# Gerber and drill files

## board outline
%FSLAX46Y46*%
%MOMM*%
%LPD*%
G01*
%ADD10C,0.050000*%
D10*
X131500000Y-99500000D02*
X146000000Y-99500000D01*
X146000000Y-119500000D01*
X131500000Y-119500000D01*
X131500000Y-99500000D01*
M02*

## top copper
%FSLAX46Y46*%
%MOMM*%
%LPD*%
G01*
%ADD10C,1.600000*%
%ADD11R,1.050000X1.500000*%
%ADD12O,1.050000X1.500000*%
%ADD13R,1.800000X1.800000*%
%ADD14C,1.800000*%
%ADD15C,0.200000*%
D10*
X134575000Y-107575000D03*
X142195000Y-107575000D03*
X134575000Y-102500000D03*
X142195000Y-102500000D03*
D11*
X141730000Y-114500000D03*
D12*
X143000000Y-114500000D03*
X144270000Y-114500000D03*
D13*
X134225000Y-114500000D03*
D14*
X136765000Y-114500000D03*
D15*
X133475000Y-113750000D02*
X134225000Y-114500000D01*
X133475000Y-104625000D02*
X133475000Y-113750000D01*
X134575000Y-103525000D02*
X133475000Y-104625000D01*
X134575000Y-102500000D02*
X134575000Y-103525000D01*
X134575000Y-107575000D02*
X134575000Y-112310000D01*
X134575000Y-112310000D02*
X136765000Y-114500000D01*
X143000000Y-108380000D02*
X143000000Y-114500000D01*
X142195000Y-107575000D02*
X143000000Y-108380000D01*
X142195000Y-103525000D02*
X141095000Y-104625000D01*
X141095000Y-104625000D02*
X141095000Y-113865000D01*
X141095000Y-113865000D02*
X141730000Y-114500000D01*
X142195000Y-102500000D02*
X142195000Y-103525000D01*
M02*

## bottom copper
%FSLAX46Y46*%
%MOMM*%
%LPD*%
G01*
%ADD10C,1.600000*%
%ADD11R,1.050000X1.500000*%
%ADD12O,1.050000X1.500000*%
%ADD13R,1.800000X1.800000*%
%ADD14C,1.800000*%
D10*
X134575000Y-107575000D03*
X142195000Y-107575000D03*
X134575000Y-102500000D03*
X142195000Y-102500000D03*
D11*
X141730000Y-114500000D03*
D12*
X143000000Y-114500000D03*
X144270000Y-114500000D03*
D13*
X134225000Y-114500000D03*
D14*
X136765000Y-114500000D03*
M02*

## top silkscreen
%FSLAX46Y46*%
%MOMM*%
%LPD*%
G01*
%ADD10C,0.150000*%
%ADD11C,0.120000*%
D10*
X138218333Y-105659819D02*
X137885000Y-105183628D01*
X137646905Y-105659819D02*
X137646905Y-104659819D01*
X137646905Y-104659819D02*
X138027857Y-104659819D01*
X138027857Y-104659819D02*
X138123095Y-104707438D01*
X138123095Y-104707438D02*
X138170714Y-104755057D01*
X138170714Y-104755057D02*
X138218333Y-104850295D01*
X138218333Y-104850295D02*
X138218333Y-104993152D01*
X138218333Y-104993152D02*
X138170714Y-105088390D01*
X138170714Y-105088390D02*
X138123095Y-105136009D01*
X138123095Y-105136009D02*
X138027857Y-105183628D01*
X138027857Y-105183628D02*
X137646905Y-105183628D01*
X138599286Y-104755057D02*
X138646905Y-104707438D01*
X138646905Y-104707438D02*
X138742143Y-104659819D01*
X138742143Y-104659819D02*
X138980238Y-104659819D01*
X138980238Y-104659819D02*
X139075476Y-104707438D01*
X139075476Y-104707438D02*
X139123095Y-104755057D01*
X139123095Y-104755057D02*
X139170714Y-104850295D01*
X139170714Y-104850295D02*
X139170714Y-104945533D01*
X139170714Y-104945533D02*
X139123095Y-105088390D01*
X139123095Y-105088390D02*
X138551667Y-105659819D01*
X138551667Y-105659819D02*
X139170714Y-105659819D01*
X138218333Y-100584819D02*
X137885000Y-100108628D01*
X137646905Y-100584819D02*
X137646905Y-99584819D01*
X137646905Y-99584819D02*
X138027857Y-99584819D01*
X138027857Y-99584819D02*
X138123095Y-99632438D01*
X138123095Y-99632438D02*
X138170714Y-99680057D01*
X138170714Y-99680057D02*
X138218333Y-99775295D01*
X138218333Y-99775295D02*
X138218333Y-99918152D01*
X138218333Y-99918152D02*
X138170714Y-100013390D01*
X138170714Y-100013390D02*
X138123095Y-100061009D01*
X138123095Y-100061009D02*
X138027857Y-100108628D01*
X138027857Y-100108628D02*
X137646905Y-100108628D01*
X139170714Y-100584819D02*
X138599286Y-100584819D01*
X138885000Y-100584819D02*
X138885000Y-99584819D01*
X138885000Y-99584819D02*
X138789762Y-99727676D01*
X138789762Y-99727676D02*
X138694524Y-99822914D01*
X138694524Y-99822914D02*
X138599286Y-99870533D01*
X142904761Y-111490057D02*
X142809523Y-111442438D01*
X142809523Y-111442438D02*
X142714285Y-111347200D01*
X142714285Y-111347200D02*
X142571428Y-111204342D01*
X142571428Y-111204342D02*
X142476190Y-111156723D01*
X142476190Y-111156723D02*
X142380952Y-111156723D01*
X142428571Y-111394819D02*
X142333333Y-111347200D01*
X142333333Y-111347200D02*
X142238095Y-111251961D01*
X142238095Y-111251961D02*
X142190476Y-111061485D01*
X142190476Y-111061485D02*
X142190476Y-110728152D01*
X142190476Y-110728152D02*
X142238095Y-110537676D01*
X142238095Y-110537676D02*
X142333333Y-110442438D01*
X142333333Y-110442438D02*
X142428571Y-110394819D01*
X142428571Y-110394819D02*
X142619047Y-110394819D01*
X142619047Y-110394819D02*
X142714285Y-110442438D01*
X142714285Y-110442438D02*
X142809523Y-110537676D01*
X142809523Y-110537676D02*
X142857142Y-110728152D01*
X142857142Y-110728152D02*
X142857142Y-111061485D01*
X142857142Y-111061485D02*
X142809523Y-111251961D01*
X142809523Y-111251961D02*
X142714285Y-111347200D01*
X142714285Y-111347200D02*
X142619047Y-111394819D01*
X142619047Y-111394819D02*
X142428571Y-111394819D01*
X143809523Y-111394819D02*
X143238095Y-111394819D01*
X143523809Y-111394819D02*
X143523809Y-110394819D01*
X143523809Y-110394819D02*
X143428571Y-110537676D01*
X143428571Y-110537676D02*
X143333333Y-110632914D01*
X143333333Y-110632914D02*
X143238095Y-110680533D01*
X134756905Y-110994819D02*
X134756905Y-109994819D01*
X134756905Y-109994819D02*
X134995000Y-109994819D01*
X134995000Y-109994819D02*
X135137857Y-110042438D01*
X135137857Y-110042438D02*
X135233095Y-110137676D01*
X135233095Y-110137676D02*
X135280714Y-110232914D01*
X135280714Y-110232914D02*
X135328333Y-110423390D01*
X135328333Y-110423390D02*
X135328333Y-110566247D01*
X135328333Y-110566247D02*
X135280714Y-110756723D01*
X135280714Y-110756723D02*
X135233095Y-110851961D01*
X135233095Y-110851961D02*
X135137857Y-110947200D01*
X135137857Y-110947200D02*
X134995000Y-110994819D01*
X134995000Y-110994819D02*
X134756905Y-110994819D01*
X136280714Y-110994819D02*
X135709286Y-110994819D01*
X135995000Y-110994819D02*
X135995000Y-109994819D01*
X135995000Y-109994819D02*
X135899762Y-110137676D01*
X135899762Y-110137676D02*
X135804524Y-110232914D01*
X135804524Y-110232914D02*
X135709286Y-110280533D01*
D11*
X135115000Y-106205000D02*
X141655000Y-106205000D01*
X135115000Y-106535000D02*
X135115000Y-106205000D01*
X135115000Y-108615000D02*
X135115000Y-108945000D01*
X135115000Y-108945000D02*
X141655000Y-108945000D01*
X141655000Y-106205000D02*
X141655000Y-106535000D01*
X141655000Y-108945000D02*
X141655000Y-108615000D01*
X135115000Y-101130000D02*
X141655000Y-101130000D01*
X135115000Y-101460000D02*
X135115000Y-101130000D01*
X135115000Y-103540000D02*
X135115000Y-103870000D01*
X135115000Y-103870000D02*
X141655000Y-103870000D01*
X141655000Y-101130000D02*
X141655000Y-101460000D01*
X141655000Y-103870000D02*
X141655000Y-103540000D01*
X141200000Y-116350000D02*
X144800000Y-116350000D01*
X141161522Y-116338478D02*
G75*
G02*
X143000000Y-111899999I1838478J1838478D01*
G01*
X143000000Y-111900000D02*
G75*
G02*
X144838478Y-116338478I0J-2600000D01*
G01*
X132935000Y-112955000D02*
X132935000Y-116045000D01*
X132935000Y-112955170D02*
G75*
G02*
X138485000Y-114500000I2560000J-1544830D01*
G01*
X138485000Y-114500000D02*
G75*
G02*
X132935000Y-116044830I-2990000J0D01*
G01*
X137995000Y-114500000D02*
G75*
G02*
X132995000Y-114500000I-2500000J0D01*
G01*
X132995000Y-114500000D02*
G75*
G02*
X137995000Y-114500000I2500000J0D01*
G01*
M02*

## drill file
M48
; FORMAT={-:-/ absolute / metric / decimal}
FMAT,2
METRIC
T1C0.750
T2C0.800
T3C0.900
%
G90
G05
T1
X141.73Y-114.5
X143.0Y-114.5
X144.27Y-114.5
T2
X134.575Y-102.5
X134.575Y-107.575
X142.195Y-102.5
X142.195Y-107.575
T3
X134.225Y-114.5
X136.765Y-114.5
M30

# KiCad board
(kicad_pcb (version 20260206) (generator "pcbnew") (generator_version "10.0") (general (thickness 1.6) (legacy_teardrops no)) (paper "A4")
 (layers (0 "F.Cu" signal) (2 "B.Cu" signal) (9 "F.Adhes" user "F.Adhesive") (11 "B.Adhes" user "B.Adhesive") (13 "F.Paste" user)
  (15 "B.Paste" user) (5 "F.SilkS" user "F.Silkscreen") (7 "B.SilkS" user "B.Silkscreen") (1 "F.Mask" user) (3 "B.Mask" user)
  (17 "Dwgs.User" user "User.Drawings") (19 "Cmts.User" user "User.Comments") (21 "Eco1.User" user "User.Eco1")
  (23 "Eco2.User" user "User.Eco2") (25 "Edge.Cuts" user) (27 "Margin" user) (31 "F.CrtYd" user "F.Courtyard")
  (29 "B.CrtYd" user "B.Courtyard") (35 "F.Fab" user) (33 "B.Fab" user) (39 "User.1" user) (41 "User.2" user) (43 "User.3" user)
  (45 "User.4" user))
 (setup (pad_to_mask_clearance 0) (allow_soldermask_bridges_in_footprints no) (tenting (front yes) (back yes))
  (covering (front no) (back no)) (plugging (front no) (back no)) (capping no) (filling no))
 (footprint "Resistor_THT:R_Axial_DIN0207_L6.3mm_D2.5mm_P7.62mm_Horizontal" (layer "F.Cu") (at 134.575 107.575)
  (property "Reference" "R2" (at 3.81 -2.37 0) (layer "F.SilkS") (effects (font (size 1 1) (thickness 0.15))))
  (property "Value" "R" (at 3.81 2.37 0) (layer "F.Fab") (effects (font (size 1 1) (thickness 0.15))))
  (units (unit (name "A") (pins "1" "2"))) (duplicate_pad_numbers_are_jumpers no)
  (fp_line (start 0.54 -1.37) (end 7.08 -1.37) (stroke (width 0.12) (type solid)) (layer "F.SilkS"))
  (fp_line (start 0.54 -1.04) (end 0.54 -1.37) (stroke (width 0.12) (type solid)) (layer "F.SilkS"))
  (fp_line (start 0.54 1.04) (end 0.54 1.37) (stroke (width 0.12) (type solid)) (layer "F.SilkS"))
  (fp_line (start 0.54 1.37) (end 7.08 1.37) (stroke (width 0.12) (type solid)) (layer "F.SilkS"))
  (fp_line (start 7.08 -1.37) (end 7.08 -1.04) (stroke (width 0.12) (type solid)) (layer "F.SilkS"))
  (fp_line (start 7.08 1.37) (end 7.08 1.04) (stroke (width 0.12) (type solid)) (layer "F.SilkS"))
  (pad "1" thru_hole circle (at 0 0) (size 1.6 1.6) (drill 0.8) (layers "*.Cu" "*.Mask") (remove_unused_layers no) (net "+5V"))
  (pad "2" thru_hole circle (at 7.62 0) (size 1.6 1.6) (drill 0.8) (layers "*.Cu" "*.Mask") (remove_unused_layers no) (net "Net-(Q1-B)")))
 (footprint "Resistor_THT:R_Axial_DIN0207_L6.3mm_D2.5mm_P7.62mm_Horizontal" (layer "F.Cu") (at 134.575 102.5)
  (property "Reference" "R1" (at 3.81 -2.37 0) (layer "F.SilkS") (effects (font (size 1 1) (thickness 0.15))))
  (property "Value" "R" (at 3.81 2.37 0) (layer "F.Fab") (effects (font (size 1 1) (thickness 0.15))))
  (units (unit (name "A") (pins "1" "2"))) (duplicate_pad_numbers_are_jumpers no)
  (fp_line (start 0.54 -1.37) (end 7.08 -1.37) (stroke (width 0.12) (type solid)) (layer "F.SilkS"))
  (fp_line (start 0.54 -1.04) (end 0.54 -1.37) (stroke (width 0.12) (type solid)) (layer "F.SilkS"))
  (fp_line (start 0.54 1.04) (end 0.54 1.37) (stroke (width 0.12) (type solid)) (layer "F.SilkS"))
  (fp_line (start 0.54 1.37) (end 7.08 1.37) (stroke (width 0.12) (type solid)) (layer "F.SilkS"))
  (fp_line (start 7.08 -1.37) (end 7.08 -1.04) (stroke (width 0.12) (type solid)) (layer "F.SilkS"))
  (fp_line (start 7.08 1.37) (end 7.08 1.04) (stroke (width 0.12) (type solid)) (layer "F.SilkS"))
  (pad "1" thru_hole circle (at 0 0) (size 1.6 1.6) (drill 0.8) (layers "*.Cu" "*.Mask") (remove_unused_layers no) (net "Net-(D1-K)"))
  (pad "2" thru_hole circle (at 7.62 0) (size 1.6 1.6) (drill 0.8) (layers "*.Cu" "*.Mask") (remove_unused_layers no) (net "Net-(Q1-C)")))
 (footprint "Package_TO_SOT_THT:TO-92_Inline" (layer "F.Cu") (at 141.73 114.5)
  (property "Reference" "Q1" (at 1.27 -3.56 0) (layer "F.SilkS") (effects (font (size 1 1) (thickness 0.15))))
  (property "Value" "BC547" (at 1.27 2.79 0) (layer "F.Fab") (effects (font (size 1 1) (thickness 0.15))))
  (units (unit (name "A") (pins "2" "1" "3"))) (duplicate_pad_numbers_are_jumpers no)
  (fp_line (start -0.53 1.85) (end 3.07 1.85) (stroke (width 0.12) (type solid)) (layer "F.SilkS"))
  (fp_arc (start -0.568478 1.838478) (mid -1.132087 -0.994977) (end 1.27 -2.6) (stroke (width 0.12) (type solid)) (layer "F.SilkS"))
  (fp_arc (start 1.27 -2.6) (mid 3.672087 -0.994977) (end 3.108478 1.838478) (stroke (width 0.12) (type solid)) (layer "F.SilkS"))
  (pad "1" thru_hole rect (at 0 0) (size 1.05 1.5) (drill 0.75) (layers "*.Cu" "*.Mask") (remove_unused_layers no) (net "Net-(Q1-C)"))
  (pad "2" thru_hole oval (at 1.27 0) (size 1.05 1.5) (drill 0.75) (layers "*.Cu" "*.Mask") (remove_unused_layers no) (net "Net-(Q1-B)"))
  (pad "3" thru_hole oval (at 2.54 0) (size 1.05 1.5) (drill 0.75) (layers "*.Cu" "*.Mask") (remove_unused_layers no) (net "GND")))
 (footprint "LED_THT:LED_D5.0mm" (layer "F.Cu") (at 134.225 114.5)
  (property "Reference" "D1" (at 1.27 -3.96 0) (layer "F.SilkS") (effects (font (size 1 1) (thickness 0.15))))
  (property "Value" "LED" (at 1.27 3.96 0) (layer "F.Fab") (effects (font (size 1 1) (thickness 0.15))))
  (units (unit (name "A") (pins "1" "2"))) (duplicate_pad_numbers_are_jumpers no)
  (fp_line (start -1.29 -1.545) (end -1.29 1.545) (stroke (width 0.12) (type solid)) (layer "F.SilkS"))
  (fp_arc (start -1.29 -1.54483) (mid 2.071779 -2.880495) (end 4.26 0) (stroke (width 0.12) (type solid)) (layer "F.SilkS"))
  (fp_arc (start 4.26 0) (mid 2.071779 2.880495) (end -1.29 1.54483) (stroke (width 0.12) (type solid)) (layer "F.SilkS"))
  (fp_circle (center 1.27 0) (end 3.77 0) (stroke (width 0.12) (type solid)) (fill no) (layer "F.SilkS"))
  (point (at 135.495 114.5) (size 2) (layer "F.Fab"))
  (pad "1" thru_hole rect (at 0 0) (size 1.8 1.8) (drill 0.9) (layers "*.Cu" "*.Mask") (remove_unused_layers no) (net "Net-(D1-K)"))
  (pad "2" thru_hole circle (at 2.54 0) (size 1.8 1.8) (drill 0.9) (layers "*.Cu" "*.Mask") (remove_unused_layers no) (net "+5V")))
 (gr_rect (start 131.5 99.5) (end 146 119.5) (stroke (width 0.05) (type default)) (fill no) (layer "Edge.Cuts"))
 (segment (start 133.475 113.75) (end 134.225 114.5) (width 0.2) (layer "F.Cu") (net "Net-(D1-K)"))
 (segment (start 133.475 104.625) (end 133.475 113.75) (width 0.2) (layer "F.Cu") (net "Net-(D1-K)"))
 (segment (start 134.575 103.525) (end 133.475 104.625) (width 0.2) (layer "F.Cu") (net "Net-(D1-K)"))
 (segment (start 134.575 102.5) (end 134.575 103.525) (width 0.2) (layer "F.Cu") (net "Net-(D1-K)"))
 (segment (start 134.575 107.575) (end 134.575 112.31) (width 0.2) (layer "F.Cu") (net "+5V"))
 (segment (start 134.575 112.31) (end 136.765 114.5) (width 0.2) (layer "F.Cu") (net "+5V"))
 (segment (start 143 108.38) (end 143 114.5) (width 0.2) (layer "F.Cu") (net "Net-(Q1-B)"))
 (segment (start 142.195 107.575) (end 143 108.38) (width 0.2) (layer "F.Cu") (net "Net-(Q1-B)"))
 (segment (start 142.195 103.525) (end 141.095 104.625) (width 0.2) (layer "F.Cu") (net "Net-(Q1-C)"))
 (segment (start 141.095 104.625) (end 141.095 113.865) (width 0.2) (layer "F.Cu") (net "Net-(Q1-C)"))
 (segment (start 141.095 113.865) (end 141.73 114.5) (width 0.2) (layer "F.Cu") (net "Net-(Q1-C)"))
 (segment (start 142.195 102.5) (end 142.195 103.525) (width 0.2) (layer "F.Cu") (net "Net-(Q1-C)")))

